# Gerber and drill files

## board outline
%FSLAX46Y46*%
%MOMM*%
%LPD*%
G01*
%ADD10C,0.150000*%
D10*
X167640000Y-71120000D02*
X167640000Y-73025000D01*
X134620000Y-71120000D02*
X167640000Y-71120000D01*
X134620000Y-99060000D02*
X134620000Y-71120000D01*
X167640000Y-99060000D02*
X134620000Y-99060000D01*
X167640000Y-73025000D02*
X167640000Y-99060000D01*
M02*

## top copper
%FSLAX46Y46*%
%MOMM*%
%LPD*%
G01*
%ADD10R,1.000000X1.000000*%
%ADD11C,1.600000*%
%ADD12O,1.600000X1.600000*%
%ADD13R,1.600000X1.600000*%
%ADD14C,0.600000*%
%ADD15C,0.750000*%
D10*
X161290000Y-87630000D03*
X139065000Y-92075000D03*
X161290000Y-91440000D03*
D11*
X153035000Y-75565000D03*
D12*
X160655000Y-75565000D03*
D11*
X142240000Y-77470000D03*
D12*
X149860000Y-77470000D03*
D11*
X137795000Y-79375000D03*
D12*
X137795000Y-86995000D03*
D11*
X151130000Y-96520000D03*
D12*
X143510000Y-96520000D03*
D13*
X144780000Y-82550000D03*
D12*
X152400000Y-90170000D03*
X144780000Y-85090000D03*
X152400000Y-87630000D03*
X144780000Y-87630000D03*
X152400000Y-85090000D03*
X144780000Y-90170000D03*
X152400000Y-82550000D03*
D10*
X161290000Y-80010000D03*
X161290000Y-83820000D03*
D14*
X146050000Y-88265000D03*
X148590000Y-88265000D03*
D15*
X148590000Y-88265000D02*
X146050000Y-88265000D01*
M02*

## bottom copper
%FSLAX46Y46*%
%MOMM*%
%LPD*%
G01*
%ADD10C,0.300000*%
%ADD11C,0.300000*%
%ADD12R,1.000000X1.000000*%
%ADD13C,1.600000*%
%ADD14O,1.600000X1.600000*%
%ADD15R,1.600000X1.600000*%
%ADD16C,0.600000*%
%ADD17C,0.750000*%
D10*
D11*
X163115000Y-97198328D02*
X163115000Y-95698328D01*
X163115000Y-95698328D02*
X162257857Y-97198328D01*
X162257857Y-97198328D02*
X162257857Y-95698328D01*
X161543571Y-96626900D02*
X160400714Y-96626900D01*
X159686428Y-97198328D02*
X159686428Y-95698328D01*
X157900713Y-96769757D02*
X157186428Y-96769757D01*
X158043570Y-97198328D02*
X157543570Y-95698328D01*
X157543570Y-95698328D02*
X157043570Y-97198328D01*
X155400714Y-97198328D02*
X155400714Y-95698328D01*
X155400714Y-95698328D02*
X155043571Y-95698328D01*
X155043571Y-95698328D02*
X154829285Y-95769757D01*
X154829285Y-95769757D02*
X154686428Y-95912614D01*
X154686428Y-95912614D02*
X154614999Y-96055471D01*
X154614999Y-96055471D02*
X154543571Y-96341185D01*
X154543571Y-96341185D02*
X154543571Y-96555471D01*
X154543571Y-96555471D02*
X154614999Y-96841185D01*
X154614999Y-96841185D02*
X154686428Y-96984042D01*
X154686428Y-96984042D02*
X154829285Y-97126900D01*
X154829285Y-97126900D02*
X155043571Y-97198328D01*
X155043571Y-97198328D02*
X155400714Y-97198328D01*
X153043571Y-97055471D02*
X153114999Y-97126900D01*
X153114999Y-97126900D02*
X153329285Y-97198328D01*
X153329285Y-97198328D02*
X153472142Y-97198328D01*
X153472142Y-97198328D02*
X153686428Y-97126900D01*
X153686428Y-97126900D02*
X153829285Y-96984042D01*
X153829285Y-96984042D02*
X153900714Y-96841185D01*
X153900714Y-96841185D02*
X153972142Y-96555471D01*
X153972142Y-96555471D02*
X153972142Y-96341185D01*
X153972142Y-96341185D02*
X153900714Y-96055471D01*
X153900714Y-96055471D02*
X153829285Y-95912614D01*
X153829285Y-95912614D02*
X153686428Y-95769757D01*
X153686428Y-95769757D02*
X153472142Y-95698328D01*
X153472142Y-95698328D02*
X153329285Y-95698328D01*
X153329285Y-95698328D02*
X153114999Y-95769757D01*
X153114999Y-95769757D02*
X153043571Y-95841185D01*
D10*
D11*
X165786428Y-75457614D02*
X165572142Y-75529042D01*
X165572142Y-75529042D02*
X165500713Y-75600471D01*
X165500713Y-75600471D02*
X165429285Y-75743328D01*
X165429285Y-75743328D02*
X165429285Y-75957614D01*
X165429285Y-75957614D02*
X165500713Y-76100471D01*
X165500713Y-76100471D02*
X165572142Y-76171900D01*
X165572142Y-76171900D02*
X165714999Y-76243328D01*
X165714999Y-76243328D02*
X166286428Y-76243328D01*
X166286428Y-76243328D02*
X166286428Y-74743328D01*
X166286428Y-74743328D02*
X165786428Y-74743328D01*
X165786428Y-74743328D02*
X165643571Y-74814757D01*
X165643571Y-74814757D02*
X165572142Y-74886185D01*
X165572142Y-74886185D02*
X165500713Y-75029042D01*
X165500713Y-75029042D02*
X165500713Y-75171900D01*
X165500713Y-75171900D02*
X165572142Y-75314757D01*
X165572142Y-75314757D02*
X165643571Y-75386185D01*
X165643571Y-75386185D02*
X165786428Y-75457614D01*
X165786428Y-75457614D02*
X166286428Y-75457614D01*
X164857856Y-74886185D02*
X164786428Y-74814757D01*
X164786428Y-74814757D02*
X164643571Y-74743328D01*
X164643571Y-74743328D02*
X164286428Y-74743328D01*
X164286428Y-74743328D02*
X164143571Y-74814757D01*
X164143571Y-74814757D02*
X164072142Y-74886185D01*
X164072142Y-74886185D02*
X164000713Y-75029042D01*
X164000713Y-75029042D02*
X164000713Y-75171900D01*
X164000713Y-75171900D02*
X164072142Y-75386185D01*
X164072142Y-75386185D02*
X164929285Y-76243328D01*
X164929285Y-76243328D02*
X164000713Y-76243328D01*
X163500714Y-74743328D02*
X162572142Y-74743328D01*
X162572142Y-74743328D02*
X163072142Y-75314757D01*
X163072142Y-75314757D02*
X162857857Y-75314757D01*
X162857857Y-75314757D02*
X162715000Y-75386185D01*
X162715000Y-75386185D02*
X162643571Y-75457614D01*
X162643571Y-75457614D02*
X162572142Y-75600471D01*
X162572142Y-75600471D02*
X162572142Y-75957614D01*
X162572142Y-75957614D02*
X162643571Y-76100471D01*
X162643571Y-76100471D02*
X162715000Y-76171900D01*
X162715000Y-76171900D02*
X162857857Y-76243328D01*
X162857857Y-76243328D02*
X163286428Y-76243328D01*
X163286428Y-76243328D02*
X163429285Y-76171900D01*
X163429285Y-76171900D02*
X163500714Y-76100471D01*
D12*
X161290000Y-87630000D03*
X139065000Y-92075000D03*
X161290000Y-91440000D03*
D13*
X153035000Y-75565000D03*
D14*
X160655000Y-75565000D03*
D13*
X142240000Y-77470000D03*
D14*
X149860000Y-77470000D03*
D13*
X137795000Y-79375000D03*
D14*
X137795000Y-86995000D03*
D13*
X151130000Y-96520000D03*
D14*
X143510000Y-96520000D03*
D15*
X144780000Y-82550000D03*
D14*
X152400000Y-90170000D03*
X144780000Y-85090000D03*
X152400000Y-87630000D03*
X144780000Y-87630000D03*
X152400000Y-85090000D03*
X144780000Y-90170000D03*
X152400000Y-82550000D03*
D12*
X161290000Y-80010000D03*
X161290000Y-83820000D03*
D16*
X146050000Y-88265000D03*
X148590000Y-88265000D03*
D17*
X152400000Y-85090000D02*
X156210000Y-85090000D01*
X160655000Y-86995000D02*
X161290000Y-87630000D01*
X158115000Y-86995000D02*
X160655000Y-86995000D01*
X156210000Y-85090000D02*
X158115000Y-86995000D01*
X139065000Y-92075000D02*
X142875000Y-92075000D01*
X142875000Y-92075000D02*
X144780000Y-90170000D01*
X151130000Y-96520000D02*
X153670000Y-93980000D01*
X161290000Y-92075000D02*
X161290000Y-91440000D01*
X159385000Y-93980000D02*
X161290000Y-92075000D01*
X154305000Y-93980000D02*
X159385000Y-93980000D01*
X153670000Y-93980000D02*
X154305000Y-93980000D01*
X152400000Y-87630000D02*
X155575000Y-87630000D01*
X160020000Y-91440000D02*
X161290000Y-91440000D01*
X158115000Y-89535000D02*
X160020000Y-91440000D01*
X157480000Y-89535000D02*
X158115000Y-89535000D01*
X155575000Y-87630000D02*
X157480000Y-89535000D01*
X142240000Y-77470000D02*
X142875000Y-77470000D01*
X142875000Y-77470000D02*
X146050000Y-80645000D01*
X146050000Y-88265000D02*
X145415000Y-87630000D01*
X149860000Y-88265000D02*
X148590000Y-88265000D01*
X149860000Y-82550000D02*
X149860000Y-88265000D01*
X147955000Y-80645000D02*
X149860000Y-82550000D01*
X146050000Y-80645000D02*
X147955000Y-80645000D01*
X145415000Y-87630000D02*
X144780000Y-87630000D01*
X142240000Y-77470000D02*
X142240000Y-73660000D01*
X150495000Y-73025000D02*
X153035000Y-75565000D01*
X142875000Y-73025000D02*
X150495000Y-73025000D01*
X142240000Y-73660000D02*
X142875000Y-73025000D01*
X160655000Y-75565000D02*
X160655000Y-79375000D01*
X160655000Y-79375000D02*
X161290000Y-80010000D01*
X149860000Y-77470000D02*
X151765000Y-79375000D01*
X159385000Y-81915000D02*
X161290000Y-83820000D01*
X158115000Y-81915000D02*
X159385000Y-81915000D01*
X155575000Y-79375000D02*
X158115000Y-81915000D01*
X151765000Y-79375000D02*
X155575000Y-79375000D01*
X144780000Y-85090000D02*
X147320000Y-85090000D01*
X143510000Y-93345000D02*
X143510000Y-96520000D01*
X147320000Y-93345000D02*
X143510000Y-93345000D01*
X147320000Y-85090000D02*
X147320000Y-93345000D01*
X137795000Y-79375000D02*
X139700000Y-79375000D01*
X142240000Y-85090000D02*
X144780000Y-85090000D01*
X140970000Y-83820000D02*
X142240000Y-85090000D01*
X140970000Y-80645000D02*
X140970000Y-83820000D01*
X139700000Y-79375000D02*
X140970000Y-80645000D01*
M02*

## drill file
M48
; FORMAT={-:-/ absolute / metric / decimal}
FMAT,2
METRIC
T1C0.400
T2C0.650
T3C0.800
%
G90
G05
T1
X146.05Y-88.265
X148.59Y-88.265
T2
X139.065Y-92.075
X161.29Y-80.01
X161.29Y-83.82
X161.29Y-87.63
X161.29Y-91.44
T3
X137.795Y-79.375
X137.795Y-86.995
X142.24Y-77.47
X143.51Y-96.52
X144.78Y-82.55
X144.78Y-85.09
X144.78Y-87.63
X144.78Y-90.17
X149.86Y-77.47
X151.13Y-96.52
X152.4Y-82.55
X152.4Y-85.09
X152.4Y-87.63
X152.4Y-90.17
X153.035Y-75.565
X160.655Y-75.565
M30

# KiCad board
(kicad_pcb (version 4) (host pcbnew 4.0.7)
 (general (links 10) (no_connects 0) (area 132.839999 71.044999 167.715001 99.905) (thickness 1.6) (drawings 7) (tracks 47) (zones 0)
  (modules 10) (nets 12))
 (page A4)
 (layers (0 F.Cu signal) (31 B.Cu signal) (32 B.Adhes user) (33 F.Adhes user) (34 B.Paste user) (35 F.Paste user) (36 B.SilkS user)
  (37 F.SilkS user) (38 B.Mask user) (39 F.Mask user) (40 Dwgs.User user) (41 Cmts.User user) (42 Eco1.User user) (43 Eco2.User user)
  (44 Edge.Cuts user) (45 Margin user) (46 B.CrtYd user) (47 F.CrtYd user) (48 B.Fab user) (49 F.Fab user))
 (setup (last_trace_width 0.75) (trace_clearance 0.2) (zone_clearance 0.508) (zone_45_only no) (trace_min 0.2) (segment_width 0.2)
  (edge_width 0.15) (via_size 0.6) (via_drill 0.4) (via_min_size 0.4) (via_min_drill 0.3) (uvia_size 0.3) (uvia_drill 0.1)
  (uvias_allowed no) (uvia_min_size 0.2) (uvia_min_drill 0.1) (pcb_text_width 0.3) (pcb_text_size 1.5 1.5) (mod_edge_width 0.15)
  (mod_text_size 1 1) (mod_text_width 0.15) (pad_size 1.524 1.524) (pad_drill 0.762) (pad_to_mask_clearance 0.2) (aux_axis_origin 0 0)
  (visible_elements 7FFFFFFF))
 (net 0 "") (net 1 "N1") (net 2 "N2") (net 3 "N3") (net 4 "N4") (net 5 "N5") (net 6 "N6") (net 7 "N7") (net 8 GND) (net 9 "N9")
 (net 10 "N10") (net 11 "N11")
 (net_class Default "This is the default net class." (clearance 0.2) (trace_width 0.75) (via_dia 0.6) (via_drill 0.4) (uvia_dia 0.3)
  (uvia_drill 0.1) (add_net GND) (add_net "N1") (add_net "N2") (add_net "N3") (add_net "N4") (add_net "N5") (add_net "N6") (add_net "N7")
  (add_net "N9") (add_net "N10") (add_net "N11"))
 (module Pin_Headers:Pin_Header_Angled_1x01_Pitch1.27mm (layer F.Cu) (at 161.29 87.63)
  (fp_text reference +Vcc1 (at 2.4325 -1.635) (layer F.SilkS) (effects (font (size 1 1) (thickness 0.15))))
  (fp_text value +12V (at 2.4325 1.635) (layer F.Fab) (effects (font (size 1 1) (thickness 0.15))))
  (pad 1 thru_hole rect (at 0 0) (size 1 1) (drill 0.65) (layers *.Cu *.Mask) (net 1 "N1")))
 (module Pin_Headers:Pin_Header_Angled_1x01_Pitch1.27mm (layer F.Cu) (at 139.065 92.075 180)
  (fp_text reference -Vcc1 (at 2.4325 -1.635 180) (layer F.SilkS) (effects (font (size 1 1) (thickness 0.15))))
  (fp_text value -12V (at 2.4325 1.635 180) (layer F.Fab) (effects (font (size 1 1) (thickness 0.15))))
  (pad 1 thru_hole rect (at 0 0 180) (size 1 1) (drill 0.65) (layers *.Cu *.Mask) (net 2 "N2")))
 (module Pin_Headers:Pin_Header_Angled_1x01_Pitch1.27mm (layer F.Cu) (at 161.29 91.44)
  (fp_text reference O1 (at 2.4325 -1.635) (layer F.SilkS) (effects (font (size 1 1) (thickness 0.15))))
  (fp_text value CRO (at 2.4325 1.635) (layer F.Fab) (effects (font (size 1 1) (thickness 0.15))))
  (pad 1 thru_hole rect (at 0 0) (size 1 1) (drill 0.65) (layers *.Cu *.Mask) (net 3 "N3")))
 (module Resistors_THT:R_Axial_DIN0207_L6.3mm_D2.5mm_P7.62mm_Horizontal (layer F.Cu) (at 153.035 75.565)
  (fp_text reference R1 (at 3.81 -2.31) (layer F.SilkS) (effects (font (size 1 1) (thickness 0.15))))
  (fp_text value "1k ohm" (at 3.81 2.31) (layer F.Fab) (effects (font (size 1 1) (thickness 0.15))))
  (pad 1 thru_hole circle (at 0 0) (size 1.6 1.6) (drill 0.8) (layers *.Cu *.Mask) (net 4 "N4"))
  (pad 2 thru_hole oval (at 7.62 0) (size 1.6 1.6) (drill 0.8) (layers *.Cu *.Mask) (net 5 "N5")))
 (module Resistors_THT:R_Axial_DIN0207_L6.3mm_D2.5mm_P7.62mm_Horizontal (layer F.Cu) (at 142.24 77.47)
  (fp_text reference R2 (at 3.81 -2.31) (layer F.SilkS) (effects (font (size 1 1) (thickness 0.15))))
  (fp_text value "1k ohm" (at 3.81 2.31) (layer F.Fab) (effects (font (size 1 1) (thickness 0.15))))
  (pad 1 thru_hole circle (at 0 0) (size 1.6 1.6) (drill 0.8) (layers *.Cu *.Mask) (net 4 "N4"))
  (pad 2 thru_hole oval (at 7.62 0) (size 1.6 1.6) (drill 0.8) (layers *.Cu *.Mask) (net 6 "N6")))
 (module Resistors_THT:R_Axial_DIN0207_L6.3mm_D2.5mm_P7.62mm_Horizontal (layer F.Cu) (at 137.795 79.375 270)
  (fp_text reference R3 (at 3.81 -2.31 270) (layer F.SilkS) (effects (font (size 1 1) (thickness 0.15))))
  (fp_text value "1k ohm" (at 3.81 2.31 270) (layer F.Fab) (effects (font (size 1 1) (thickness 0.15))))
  (pad 1 thru_hole circle (at 0 0 270) (size 1.6 1.6) (drill 0.8) (layers *.Cu *.Mask) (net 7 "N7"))
  (pad 2 thru_hole oval (at 7.62 0 270) (size 1.6 1.6) (drill 0.8) (layers *.Cu *.Mask) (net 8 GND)))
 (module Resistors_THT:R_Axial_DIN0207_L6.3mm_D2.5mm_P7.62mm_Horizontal (layer F.Cu) (at 151.13 96.52 180)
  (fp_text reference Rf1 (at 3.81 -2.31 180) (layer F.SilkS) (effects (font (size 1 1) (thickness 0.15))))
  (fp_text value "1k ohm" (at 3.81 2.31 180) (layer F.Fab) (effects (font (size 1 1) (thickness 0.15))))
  (pad 1 thru_hole circle (at 0 0 180) (size 1.6 1.6) (drill 0.8) (layers *.Cu *.Mask) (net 3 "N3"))
  (pad 2 thru_hole oval (at 7.62 0 180) (size 1.6 1.6) (drill 0.8) (layers *.Cu *.Mask) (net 7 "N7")))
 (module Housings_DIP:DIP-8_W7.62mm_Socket (layer F.Cu) (at 144.78 82.55)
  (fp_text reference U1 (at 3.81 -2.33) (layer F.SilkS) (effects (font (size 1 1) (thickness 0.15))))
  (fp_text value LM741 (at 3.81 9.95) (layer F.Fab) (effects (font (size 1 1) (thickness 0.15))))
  (pad 1 thru_hole rect (at 0 0) (size 1.6 1.6) (drill 0.8) (layers *.Cu *.Mask) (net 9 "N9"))
  (pad 5 thru_hole oval (at 7.62 7.62) (size 1.6 1.6) (drill 0.8) (layers *.Cu *.Mask) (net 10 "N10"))
  (pad 2 thru_hole oval (at 0 2.54) (size 1.6 1.6) (drill 0.8) (layers *.Cu *.Mask) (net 7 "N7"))
  (pad 6 thru_hole oval (at 7.62 5.08) (size 1.6 1.6) (drill 0.8) (layers *.Cu *.Mask) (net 3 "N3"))
  (pad 3 thru_hole oval (at 0 5.08) (size 1.6 1.6) (drill 0.8) (layers *.Cu *.Mask) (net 4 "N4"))
  (pad 7 thru_hole oval (at 7.62 2.54) (size 1.6 1.6) (drill 0.8) (layers *.Cu *.Mask) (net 1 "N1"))
  (pad 4 thru_hole oval (at 0 7.62) (size 1.6 1.6) (drill 0.8) (layers *.Cu *.Mask) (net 2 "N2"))
  (pad 8 thru_hole oval (at 7.62 0) (size 1.6 1.6) (drill 0.8) (layers *.Cu *.Mask) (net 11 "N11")))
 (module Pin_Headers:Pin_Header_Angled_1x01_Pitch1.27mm (layer F.Cu) (at 161.29 80.01)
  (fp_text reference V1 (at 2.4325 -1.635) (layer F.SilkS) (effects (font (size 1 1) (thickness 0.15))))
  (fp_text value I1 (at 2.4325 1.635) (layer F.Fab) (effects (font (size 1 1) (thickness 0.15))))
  (pad 1 thru_hole rect (at 0 0) (size 1 1) (drill 0.65) (layers *.Cu *.Mask) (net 5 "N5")))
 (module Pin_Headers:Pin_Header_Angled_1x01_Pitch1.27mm (layer F.Cu) (at 161.29 83.82)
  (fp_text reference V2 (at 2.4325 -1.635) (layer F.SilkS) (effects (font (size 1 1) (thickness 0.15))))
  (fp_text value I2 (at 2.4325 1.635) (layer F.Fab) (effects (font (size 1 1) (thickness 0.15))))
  (pad 1 thru_hole rect (at 0 0) (size 1 1) (drill 0.65) (layers *.Cu *.Mask) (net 6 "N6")))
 (gr_line (start 167.64 71.12) (end 167.64 73.025) (angle 90) (layer Edge.Cuts) (width 0.15))
 (gr_line (start 134.62 71.12) (end 167.64 71.12) (angle 90) (layer Edge.Cuts) (width 0.15))
 (gr_line (start 134.62 99.06) (end 134.62 71.12) (angle 90) (layer Edge.Cuts) (width 0.15))
 (gr_line (start 167.64 99.06) (end 134.62 99.06) (angle 90) (layer Edge.Cuts) (width 0.15))
 (gr_line (start 167.64 73.025) (end 167.64 99.06) (angle 90) (layer Edge.Cuts) (width 0.15))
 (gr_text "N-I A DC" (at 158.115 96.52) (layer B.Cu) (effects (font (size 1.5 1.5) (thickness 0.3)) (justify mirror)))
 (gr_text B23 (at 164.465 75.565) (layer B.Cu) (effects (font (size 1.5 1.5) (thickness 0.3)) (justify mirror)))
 (segment (start 152.4 85.09) (end 156.21 85.09) (width 0.75) (layer B.Cu) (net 1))
 (segment (start 160.655 86.995) (end 161.29 87.63) (width 0.75) (layer B.Cu) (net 1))
 (segment (start 158.115 86.995) (end 160.655 86.995) (width 0.75) (layer B.Cu) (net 1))
 (segment (start 156.21 85.09) (end 158.115 86.995) (width 0.75) (layer B.Cu) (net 1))
 (segment (start 139.065 92.075) (end 142.875 92.075) (width 0.75) (layer B.Cu) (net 2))
 (segment (start 142.875 92.075) (end 144.78 90.17) (width 0.75) (layer B.Cu) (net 2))
 (segment (start 151.13 96.52) (end 153.67 93.98) (width 0.75) (layer B.Cu) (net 3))
 (segment (start 161.29 92.075) (end 161.29 91.44) (width 0.75) (layer B.Cu) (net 3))
 (segment (start 159.385 93.98) (end 161.29 92.075) (width 0.75) (layer B.Cu) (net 3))
 (segment (start 154.305 93.98) (end 159.385 93.98) (width 0.75) (layer B.Cu) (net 3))
 (segment (start 153.67 93.98) (end 154.305 93.98) (width 0.75) (layer B.Cu) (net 3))
 (segment (start 152.4 87.63) (end 155.575 87.63) (width 0.75) (layer B.Cu) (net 3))
 (segment (start 160.02 91.44) (end 161.29 91.44) (width 0.75) (layer B.Cu) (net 3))
 (segment (start 158.115 89.535) (end 160.02 91.44) (width 0.75) (layer B.Cu) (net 3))
 (segment (start 157.48 89.535) (end 158.115 89.535) (width 0.75) (layer B.Cu) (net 3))
 (segment (start 155.575 87.63) (end 157.48 89.535) (width 0.75) (layer B.Cu) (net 3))
 (segment (start 142.24 77.47) (end 142.875 77.47) (width 0.75) (layer B.Cu) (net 4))
 (segment (start 142.875 77.47) (end 146.05 80.645) (width 0.75) (layer B.Cu) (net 4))
 (segment (start 146.05 88.265) (end 145.415 87.63) (width 0.75) (layer B.Cu) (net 4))
 (via (at 146.05 88.265) (size 0.6) (drill 0.4) (layers F.Cu B.Cu) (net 4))
 (segment (start 148.59 88.265) (end 146.05 88.265) (width 0.75) (layer F.Cu) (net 4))
 (via (at 148.59 88.265) (size 0.6) (drill 0.4) (layers F.Cu B.Cu) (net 4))
 (segment (start 149.86 88.265) (end 148.59 88.265) (width 0.75) (layer B.Cu) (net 4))
 (segment (start 149.86 82.55) (end 149.86 88.265) (width 0.75) (layer B.Cu) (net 4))
 (segment (start 147.955 80.645) (end 149.86 82.55) (width 0.75) (layer B.Cu) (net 4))
 (segment (start 146.05 80.645) (end 147.955 80.645) (width 0.75) (layer B.Cu) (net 4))
 (segment (start 145.415 87.63) (end 144.78 87.63) (width 0.75) (layer B.Cu) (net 4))
 (segment (start 142.24 77.47) (end 142.24 73.66) (width 0.75) (layer B.Cu) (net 4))
 (segment (start 150.495 73.025) (end 153.035 75.565) (width 0.75) (layer B.Cu) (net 4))
 (segment (start 142.875 73.025) (end 150.495 73.025) (width 0.75) (layer B.Cu) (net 4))
 (segment (start 142.24 73.66) (end 142.875 73.025) (width 0.75) (layer B.Cu) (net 4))
 (segment (start 160.655 75.565) (end 160.655 79.375) (width 0.75) (layer B.Cu) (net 5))
 (segment (start 160.655 79.375) (end 161.29 80.01) (width 0.75) (layer B.Cu) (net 5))
 (segment (start 149.86 77.47) (end 151.765 79.375) (width 0.75) (layer B.Cu) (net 6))
 (segment (start 159.385 81.915) (end 161.29 83.82) (width 0.75) (layer B.Cu) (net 6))
 (segment (start 158.115 81.915) (end 159.385 81.915) (width 0.75) (layer B.Cu) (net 6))
 (segment (start 155.575 79.375) (end 158.115 81.915) (width 0.75) (layer B.Cu) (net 6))
 (segment (start 151.765 79.375) (end 155.575 79.375) (width 0.75) (layer B.Cu) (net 6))
 (segment (start 144.78 85.09) (end 147.32 85.09) (width 0.75) (layer B.Cu) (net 7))
 (segment (start 143.51 93.345) (end 143.51 96.52) (width 0.75) (layer B.Cu) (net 7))
 (segment (start 147.32 93.345) (end 143.51 93.345) (width 0.75) (layer B.Cu) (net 7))
 (segment (start 147.32 85.09) (end 147.32 93.345) (width 0.75) (layer B.Cu) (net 7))
 (segment (start 137.795 79.375) (end 139.7 79.375) (width 0.75) (layer B.Cu) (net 7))
 (segment (start 142.24 85.09) (end 144.78 85.09) (width 0.75) (layer B.Cu) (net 7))
 (segment (start 140.97 83.82) (end 142.24 85.09) (width 0.75) (layer B.Cu) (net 7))
 (segment (start 140.97 80.645) (end 140.97 83.82) (width 0.75) (layer B.Cu) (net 7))
 (segment (start 139.7 79.375) (end 140.97 80.645) (width 0.75) (layer B.Cu) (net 7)))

